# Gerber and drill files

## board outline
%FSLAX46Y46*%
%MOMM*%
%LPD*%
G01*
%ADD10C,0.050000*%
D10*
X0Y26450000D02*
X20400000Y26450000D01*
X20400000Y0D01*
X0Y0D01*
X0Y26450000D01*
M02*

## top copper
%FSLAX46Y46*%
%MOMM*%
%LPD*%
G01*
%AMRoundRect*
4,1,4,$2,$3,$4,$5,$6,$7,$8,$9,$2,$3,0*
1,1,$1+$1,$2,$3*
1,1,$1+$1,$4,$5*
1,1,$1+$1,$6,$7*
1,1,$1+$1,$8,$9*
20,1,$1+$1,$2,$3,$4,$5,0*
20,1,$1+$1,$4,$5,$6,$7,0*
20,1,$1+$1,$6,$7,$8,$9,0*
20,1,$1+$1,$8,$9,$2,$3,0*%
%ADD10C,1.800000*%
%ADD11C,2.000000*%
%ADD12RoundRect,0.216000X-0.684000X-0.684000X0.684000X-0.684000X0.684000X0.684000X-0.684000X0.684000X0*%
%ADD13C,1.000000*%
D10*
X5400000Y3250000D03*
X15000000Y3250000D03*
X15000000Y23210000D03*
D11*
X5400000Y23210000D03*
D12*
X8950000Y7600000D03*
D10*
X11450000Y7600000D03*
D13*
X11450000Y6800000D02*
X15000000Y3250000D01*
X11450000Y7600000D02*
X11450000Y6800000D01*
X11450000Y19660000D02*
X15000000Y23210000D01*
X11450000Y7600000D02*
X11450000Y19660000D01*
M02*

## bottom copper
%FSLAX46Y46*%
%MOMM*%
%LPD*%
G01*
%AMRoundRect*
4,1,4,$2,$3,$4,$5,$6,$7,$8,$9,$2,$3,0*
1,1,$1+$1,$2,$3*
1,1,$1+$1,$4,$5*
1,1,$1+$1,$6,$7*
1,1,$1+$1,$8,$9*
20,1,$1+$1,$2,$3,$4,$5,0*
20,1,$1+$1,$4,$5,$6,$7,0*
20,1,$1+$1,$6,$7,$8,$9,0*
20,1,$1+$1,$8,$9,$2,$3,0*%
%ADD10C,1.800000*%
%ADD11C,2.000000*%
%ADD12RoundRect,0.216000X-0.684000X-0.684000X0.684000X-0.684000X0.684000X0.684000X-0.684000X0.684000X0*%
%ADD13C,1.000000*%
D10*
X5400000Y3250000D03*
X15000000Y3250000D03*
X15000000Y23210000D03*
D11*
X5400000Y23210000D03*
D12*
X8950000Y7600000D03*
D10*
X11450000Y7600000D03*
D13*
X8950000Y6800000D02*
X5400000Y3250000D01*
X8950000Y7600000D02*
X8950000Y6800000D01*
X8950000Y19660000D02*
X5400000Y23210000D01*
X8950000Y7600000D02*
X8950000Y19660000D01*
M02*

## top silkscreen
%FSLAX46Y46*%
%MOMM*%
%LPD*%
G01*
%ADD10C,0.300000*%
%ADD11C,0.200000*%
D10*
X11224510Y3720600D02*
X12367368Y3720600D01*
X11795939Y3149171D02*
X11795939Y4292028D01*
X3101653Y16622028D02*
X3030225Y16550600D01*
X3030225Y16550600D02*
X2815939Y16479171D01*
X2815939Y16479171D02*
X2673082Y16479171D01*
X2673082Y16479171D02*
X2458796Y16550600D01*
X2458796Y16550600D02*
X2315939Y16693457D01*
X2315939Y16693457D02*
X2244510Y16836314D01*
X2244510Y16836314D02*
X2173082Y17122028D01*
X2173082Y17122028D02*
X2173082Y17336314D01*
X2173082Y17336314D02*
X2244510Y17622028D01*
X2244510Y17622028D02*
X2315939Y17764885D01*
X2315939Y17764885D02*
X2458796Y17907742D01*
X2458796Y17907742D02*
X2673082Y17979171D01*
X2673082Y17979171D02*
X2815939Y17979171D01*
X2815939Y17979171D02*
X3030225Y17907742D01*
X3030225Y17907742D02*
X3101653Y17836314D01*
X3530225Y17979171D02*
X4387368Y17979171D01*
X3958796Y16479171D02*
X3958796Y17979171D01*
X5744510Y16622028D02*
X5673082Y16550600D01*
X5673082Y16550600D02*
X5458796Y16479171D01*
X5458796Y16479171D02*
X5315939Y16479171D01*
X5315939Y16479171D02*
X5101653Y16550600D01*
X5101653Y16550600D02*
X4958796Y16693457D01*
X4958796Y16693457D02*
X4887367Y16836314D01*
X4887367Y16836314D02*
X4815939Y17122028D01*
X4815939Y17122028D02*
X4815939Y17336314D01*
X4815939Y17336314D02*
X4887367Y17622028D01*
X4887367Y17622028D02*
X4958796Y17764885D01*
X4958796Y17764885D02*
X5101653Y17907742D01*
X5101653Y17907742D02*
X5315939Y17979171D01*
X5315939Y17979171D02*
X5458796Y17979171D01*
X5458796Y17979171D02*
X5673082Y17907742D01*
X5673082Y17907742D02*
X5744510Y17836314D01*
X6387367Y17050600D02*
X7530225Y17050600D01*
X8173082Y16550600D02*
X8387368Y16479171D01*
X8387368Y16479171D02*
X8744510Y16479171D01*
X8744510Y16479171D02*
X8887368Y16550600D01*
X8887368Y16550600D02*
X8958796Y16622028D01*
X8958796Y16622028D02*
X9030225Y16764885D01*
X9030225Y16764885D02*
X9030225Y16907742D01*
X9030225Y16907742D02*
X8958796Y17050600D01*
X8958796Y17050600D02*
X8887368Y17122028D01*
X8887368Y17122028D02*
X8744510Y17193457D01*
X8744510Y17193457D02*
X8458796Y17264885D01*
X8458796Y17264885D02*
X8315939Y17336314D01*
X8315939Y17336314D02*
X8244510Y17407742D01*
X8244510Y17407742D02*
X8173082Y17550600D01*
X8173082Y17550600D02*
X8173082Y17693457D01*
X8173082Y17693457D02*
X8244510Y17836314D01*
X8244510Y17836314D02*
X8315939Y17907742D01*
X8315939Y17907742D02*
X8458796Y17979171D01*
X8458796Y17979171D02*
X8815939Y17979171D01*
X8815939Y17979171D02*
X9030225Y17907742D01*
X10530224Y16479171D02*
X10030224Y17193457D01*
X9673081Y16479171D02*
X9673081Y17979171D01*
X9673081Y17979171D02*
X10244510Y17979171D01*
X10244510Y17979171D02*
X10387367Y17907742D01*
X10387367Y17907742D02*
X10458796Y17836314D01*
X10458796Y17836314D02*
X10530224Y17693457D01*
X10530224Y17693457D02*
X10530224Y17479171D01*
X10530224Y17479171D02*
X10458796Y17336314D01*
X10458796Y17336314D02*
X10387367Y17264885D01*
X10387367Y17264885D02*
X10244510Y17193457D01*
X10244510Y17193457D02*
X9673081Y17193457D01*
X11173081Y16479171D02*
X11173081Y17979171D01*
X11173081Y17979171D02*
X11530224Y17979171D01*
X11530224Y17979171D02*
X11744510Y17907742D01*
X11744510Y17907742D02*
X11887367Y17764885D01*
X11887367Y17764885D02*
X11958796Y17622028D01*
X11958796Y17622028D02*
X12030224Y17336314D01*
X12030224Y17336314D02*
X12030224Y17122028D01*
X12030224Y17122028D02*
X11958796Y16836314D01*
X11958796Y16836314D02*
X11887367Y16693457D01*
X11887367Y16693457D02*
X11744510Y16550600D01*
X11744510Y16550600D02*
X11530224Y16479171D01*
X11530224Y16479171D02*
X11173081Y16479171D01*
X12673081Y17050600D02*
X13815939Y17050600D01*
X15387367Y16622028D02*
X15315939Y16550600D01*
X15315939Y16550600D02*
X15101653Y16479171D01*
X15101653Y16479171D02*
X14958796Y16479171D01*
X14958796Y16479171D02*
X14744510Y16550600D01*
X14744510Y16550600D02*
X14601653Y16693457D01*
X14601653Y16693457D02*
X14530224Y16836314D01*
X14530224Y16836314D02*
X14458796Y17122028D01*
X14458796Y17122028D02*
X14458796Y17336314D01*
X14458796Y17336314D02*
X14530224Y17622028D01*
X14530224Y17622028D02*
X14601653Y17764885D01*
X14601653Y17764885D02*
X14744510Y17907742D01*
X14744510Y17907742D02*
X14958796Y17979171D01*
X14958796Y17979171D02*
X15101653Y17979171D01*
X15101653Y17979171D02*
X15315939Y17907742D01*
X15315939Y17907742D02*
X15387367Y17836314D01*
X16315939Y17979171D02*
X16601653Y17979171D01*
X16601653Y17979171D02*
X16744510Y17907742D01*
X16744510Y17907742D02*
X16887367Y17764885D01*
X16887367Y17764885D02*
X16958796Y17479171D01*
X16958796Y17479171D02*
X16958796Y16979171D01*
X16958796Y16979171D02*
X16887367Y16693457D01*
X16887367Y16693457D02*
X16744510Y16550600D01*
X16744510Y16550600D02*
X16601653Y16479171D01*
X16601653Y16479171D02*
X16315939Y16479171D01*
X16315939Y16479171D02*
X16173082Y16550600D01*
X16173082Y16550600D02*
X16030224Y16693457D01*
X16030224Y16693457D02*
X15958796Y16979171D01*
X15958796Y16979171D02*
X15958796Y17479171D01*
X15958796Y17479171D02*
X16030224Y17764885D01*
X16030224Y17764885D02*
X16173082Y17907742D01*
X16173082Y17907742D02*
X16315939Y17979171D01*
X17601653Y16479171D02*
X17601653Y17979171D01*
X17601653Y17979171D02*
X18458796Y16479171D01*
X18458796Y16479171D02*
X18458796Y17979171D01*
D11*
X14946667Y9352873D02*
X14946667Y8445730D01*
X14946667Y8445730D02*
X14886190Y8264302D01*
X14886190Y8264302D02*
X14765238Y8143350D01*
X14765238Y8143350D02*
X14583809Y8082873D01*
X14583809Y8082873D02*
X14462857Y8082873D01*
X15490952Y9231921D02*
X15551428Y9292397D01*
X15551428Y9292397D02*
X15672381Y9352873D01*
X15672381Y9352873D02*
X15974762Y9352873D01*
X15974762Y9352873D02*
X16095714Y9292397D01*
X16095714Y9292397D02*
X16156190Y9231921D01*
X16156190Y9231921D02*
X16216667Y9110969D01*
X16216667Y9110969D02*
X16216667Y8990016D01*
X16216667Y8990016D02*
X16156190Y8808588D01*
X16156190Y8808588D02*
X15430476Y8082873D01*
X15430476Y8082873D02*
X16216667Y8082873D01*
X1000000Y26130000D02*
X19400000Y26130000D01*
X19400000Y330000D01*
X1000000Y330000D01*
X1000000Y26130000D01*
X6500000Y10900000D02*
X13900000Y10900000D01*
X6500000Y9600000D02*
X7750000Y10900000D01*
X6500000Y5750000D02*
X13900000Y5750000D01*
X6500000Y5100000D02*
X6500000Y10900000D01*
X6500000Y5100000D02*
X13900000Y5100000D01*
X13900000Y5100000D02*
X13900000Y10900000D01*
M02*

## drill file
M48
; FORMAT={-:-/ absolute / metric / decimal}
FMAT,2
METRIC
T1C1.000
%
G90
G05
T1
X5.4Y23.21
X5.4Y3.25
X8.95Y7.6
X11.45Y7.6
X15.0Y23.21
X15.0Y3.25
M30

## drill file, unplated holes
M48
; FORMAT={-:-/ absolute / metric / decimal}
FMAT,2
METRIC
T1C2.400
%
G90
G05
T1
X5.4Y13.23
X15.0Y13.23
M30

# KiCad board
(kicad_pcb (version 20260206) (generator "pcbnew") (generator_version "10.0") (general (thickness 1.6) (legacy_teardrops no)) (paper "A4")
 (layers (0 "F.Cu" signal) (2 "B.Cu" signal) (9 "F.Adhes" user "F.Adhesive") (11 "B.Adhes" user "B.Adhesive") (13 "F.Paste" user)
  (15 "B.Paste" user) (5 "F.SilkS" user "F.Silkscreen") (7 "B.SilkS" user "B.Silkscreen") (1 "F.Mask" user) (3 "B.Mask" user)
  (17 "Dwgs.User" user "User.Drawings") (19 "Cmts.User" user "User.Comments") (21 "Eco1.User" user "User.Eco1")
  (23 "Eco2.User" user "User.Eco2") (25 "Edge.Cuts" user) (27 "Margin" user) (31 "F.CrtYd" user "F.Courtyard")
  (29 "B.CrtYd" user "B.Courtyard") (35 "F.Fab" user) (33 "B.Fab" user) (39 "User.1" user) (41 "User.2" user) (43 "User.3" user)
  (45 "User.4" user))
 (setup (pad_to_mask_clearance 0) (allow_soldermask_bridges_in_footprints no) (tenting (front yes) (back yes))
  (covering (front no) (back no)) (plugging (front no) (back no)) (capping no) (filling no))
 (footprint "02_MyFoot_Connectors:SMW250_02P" (layer "F.Cu") (at 10.2 -7.6)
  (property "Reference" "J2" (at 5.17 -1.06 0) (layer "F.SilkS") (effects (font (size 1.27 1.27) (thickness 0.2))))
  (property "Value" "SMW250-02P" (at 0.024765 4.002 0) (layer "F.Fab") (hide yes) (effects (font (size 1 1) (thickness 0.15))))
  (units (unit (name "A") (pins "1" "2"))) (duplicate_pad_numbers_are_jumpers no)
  (fp_line (start -3.7 -3.3) (end 3.7 -3.3) (stroke (width 0.2) (type solid)) (layer "F.SilkS"))
  (fp_line (start -3.7 -2) (end -2.45 -3.3) (stroke (width 0.2) (type solid)) (layer "F.SilkS"))
  (fp_line (start -3.7 1.85) (end 3.7 1.85) (stroke (width 0.2) (type solid)) (layer "F.SilkS"))
  (fp_line (start -3.7 2.5) (end -3.7 -3.3) (stroke (width 0.2) (type solid)) (layer "F.SilkS"))
  (fp_line (start -3.7 2.5) (end 3.7 2.5) (stroke (width 0.2) (type solid)) (layer "F.SilkS"))
  (fp_line (start 3.7 2.5) (end 3.7 -3.3) (stroke (width 0.2) (type solid)) (layer "F.SilkS"))
  (pad "1" thru_hole roundrect (at -1.25 0) (size 1.8 1.8) (drill 1) (layers "*.Cu" "*.Mask") (remove_unused_layers no)
   (roundrect_rratio 0.12) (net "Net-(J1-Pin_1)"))
  (pad "2" thru_hole circle (at 1.25 0) (size 1.8 1.8) (drill 1) (layers "*.Cu" "*.Mask") (remove_unused_layers no) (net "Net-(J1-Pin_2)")
   (thermal_bridge_angle 90)))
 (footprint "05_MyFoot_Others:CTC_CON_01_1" (layer "F.Cu") (at 10.2 -13.23)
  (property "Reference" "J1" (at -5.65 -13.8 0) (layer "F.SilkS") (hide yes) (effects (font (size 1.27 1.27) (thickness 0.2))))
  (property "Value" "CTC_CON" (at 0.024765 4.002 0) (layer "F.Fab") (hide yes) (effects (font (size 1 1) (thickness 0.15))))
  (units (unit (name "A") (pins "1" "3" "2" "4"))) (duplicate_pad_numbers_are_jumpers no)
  (fp_rect (start -9.2 -12.9) (end 9.2 12.9) (stroke (width 0.2) (type default)) (fill no) (layer "F.SilkS"))
  (pad "" np_thru_hole circle (at -4.8 0) (size 2.4 2.4) (drill 2.4) (layers "*.Cu") (thermal_bridge_angle 90))
  (pad "" np_thru_hole circle (at 4.8 0) (size 2.4 2.4) (drill 2.4) (layers "*.Cu") (thermal_bridge_angle 90))
  (pad "1" thru_hole circle (at -4.8 -9.98) (size 2 2) (drill 1) (layers "*.Cu" "*.Mask") (remove_unused_layers no) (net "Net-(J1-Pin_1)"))
  (pad "2" thru_hole circle (at 4.8 -9.98) (size 1.8 1.8) (drill 1) (layers "*.Cu" "*.Mask") (remove_unused_layers no)
   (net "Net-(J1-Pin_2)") (thermal_bridge_angle 90))
  (pad "3" thru_hole circle (at 4.8 9.98) (size 1.8 1.8) (drill 1) (layers "*.Cu" "*.Mask") (remove_unused_layers no) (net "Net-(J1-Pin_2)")
   (thermal_bridge_angle 90))
  (pad "4" thru_hole circle (at -4.8 9.98) (size 1.8 1.8) (drill 1) (layers "*.Cu" "*.Mask") (remove_unused_layers no)
   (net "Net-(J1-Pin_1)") (thermal_bridge_angle 90)))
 (gr_rect (start 0 -26.45) (end 20.4 0) (stroke (width 0.05) (type solid)) (fill no) (layer "Edge.Cuts"))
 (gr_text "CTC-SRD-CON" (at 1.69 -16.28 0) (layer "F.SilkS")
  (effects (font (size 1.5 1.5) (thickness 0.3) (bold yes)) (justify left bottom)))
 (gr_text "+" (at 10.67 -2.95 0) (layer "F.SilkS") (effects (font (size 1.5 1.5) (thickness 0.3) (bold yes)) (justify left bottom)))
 (segment (start 8.95 -7.6) (end 8.95 -6.8) (width 1) (layer "B.Cu") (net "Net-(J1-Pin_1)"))
 (segment (start 8.95 -19.66) (end 5.4 -23.21) (width 1) (layer "B.Cu") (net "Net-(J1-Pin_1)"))
 (segment (start 8.95 -7.6) (end 8.95 -19.66) (width 1) (layer "B.Cu") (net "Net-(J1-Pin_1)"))
 (segment (start 8.95 -6.8) (end 5.4 -3.25) (width 1) (layer "B.Cu") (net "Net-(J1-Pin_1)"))
 (segment (start 11.45 -19.66) (end 15 -23.21) (width 1) (layer "F.Cu") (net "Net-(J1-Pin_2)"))
 (segment (start 11.45 -6.8) (end 15 -3.25) (width 1) (layer "F.Cu") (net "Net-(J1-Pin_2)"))
 (segment (start 11.45 -7.6) (end 11.45 -6.8) (width 1) (layer "F.Cu") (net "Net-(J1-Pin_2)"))
 (segment (start 11.45 -7.6) (end 11.45 -19.66) (width 1) (layer "F.Cu") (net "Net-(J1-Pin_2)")))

